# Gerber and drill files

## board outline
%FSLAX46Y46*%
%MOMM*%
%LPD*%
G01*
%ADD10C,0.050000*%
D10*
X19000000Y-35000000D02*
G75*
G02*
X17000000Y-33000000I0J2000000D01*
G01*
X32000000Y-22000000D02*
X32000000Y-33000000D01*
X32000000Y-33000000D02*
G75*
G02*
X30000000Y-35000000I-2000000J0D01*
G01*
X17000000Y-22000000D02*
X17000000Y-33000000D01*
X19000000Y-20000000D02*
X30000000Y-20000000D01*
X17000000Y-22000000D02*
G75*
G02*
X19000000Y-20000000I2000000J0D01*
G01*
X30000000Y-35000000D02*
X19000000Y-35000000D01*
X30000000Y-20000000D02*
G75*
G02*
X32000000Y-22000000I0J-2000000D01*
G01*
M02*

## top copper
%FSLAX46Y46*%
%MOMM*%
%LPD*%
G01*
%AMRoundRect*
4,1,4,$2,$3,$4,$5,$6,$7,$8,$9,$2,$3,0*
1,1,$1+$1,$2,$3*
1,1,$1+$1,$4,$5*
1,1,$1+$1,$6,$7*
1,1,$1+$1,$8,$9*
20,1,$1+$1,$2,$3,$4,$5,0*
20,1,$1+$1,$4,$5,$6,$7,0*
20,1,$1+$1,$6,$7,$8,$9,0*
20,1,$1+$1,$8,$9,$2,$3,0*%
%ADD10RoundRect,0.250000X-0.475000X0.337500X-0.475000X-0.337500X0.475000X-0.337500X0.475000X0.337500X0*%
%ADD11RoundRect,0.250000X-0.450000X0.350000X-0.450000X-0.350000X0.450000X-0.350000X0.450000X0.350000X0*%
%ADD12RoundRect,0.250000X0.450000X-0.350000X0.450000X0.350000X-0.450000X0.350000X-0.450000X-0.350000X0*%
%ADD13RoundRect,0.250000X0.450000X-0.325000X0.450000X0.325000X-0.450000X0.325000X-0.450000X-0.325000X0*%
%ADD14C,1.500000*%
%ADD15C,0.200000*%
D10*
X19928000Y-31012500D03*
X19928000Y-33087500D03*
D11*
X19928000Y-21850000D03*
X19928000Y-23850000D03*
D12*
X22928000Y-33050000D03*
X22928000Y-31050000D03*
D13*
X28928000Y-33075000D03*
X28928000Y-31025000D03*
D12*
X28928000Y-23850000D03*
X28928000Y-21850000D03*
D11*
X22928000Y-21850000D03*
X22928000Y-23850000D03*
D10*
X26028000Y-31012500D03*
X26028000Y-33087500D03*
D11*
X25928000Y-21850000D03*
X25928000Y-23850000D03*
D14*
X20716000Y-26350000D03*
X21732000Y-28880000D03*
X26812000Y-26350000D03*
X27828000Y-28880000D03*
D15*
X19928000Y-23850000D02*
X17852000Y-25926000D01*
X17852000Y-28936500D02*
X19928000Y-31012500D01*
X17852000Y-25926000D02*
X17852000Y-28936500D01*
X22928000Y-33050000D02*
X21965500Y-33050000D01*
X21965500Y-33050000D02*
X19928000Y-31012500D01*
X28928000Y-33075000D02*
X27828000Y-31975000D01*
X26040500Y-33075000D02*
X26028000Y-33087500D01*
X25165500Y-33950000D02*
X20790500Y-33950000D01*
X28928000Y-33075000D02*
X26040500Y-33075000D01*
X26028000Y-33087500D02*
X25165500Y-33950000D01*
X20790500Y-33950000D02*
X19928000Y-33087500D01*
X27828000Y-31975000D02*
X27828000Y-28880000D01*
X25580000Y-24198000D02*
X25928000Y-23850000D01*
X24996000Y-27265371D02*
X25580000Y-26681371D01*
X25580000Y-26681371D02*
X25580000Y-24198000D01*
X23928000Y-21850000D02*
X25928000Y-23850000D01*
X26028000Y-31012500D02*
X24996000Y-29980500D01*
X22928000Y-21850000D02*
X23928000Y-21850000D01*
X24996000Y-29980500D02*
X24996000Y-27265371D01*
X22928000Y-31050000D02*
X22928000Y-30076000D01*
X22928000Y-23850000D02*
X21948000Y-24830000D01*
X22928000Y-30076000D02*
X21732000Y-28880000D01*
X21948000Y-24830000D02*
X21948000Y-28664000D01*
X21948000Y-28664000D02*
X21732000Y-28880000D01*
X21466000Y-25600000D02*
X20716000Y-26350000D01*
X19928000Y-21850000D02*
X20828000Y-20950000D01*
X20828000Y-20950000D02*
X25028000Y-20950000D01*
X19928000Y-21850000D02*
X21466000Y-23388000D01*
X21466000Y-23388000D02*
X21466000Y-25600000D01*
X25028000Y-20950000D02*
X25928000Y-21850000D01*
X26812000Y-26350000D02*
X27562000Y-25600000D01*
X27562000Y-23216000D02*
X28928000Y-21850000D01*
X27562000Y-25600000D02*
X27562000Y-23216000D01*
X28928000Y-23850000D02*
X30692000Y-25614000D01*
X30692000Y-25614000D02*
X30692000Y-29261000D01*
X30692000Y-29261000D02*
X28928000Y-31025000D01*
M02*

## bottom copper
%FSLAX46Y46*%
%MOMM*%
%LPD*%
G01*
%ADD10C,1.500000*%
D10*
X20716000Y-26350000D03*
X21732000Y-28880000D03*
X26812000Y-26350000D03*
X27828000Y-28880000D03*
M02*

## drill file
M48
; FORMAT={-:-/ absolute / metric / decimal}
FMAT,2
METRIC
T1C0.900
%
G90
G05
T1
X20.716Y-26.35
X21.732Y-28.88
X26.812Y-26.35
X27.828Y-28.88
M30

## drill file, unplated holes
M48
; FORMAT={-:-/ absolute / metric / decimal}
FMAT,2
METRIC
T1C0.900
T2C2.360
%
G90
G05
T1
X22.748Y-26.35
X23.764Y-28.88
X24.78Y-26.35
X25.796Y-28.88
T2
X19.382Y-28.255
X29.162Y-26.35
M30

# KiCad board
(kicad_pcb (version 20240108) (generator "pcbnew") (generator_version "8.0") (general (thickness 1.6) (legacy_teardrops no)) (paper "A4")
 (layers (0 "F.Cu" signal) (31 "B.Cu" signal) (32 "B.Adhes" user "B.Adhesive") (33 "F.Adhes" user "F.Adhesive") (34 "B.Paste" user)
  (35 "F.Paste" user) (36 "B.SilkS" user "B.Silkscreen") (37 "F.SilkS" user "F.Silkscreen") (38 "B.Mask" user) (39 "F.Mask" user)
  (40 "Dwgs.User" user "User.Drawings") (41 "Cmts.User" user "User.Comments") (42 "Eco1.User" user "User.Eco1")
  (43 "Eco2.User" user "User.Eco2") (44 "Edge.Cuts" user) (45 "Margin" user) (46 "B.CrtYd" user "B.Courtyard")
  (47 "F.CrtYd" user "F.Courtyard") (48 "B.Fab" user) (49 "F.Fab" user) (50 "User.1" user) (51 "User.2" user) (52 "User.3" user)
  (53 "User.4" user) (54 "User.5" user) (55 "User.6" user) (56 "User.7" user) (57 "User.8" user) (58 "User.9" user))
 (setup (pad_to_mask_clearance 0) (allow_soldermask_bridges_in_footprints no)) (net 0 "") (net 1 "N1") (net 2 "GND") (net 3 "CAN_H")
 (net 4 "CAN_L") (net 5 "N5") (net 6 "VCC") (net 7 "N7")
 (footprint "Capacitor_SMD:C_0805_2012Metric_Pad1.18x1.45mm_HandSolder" (layer "F.Cu") (at 19.928 32.05 -90)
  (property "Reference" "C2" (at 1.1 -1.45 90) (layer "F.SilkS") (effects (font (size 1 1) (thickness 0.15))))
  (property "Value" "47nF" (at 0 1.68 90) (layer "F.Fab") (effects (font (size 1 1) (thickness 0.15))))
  (pad "1" smd roundrect (at -1.0375 0 270) (size 1.175 1.45) (layers "F.Cu" "F.Paste" "F.Mask") (roundrect_rratio 0.212766) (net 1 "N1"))
  (pad "2" smd roundrect (at 1.0375 0 270) (size 1.175 1.45) (layers "F.Cu" "F.Paste" "F.Mask") (roundrect_rratio 0.212766) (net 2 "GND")))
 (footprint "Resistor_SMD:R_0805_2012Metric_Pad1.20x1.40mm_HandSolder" (layer "F.Cu") (at 19.928 22.85 -90)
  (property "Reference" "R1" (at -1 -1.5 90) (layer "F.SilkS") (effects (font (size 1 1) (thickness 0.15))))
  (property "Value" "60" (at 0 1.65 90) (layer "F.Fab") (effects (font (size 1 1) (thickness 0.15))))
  (pad "1" smd roundrect (at -1 0 270) (size 1.2 1.4) (layers "F.Cu" "F.Paste" "F.Mask") (roundrect_rratio 0.208333) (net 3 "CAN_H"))
  (pad "2" smd roundrect (at 1 0 270) (size 1.2 1.4) (layers "F.Cu" "F.Paste" "F.Mask") (roundrect_rratio 0.208333) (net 1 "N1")))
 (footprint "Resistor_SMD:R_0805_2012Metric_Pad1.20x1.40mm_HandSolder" (layer "F.Cu") (at 22.928 32.05 90)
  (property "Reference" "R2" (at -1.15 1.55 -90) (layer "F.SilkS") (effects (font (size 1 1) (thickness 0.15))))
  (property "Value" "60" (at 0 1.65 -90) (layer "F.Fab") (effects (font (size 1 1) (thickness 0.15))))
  (pad "1" smd roundrect (at -1 0 90) (size 1.2 1.4) (layers "F.Cu" "F.Paste" "F.Mask") (roundrect_rratio 0.208333) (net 1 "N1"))
  (pad "2" smd roundrect (at 1 0 90) (size 1.2 1.4) (layers "F.Cu" "F.Paste" "F.Mask") (roundrect_rratio 0.208333) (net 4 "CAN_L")))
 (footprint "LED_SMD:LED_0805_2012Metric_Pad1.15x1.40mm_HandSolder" (layer "F.Cu") (at 28.928 32.05 90)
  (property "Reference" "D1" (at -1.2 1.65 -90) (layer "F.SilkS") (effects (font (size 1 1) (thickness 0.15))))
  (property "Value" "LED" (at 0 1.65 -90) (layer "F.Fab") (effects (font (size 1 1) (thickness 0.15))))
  (pad "1" smd roundrect (at -1.025 0 90) (size 1.15 1.4) (layers "F.Cu" "F.Paste" "F.Mask") (roundrect_rratio 0.217391) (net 2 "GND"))
  (pad "2" smd roundrect (at 1.025 0 90) (size 1.15 1.4) (layers "F.Cu" "F.Paste" "F.Mask") (roundrect_rratio 0.217391) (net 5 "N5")))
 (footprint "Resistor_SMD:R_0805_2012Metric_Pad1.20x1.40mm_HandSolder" (layer "F.Cu") (at 28.928 22.85 90)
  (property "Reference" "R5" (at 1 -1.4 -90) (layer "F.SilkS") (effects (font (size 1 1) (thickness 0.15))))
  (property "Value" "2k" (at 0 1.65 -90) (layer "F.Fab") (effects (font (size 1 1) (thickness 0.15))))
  (pad "1" smd roundrect (at -1 0 90) (size 1.2 1.4) (layers "F.Cu" "F.Paste" "F.Mask") (roundrect_rratio 0.208333) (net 5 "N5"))
  (pad "2" smd roundrect (at 1 0 90) (size 1.2 1.4) (layers "F.Cu" "F.Paste" "F.Mask") (roundrect_rratio 0.208333) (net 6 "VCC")))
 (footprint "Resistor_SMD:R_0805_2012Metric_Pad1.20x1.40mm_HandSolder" (layer "F.Cu") (at 22.928 22.85 -90)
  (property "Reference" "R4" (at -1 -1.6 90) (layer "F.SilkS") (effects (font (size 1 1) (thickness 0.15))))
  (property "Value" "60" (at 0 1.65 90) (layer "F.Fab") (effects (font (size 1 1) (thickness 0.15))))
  (pad "1" smd roundrect (at -1 0 270) (size 1.2 1.4) (layers "F.Cu" "F.Paste" "F.Mask") (roundrect_rratio 0.208333) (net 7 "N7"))
  (pad "2" smd roundrect (at 1 0 270) (size 1.2 1.4) (layers "F.Cu" "F.Paste" "F.Mask") (roundrect_rratio 0.208333) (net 4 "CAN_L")))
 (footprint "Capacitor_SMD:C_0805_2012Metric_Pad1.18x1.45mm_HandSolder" (layer "F.Cu") (at 26.028 32.05 -90)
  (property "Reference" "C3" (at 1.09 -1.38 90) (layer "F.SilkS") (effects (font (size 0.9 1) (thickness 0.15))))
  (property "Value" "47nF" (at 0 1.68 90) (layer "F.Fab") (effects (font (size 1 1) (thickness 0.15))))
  (pad "1" smd roundrect (at -1.0375 0 270) (size 1.175 1.45) (layers "F.Cu" "F.Paste" "F.Mask") (roundrect_rratio 0.212766) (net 7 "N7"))
  (pad "2" smd roundrect (at 1.0375 0 270) (size 1.175 1.45) (layers "F.Cu" "F.Paste" "F.Mask") (roundrect_rratio 0.212766) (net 2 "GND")))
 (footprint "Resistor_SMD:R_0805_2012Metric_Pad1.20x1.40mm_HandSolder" (layer "F.Cu") (at 25.928 22.85 -90)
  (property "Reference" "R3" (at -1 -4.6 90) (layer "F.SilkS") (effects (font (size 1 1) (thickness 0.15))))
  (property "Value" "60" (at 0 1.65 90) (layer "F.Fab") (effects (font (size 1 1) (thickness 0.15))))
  (pad "1" smd roundrect (at -1 0 270) (size 1.2 1.4) (layers "F.Cu" "F.Paste" "F.Mask") (roundrect_rratio 0.208333) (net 3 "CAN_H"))
  (pad "2" smd roundrect (at 1 0 270) (size 1.2 1.4) (layers "F.Cu" "F.Paste" "F.Mask") (roundrect_rratio 0.208333) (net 7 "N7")))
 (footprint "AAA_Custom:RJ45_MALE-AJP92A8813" (layer "B.Cu") (at 24.272 27.62 180)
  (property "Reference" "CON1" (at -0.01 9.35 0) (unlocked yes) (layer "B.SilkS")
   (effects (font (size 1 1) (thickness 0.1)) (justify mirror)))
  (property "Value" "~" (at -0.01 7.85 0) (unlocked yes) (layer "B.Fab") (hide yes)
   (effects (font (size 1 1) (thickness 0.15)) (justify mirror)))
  (pad "" np_thru_hole circle (at -4.89 1.27 180) (size 2.3 2.3) (drill 2.36) (layers "F&B.Cu" "*.Mask"))
  (pad "" np_thru_hole circle (at -1.524 -1.26 180) (size 0.9 0.9) (drill 0.9) (layers "F&B.Cu" "*.Mask"))
  (pad "" np_thru_hole circle (at -0.508 1.27 180) (size 0.9 0.9) (drill 0.9) (layers "F&B.Cu" "*.Mask"))
  (pad "" np_thru_hole circle (at 0.508 -1.26 180) (size 0.9 0.9) (drill 0.9) (layers "F&B.Cu" "*.Mask"))
  (pad "" np_thru_hole circle (at 1.524 1.27 180) (size 0.9 0.9) (drill 0.9) (layers "F&B.Cu" "*.Mask"))
  (pad "" np_thru_hole circle (at 4.89 -0.635 180) (size 2.3 2.3) (drill 2.36) (layers "F&B.Cu" "*.Mask"))
  (pad "1" thru_hole circle (at 3.556 1.27 180) (size 1.5 1.5) (drill 0.9) (layers "*.Cu" "*.Mask") (remove_unused_layers no)
   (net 3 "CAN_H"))
  (pad "2" thru_hole circle (at 2.54 -1.26 180) (size 1.5 1.5) (drill 0.9) (layers "*.Cu" "*.Mask") (remove_unused_layers no)
   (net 4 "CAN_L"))
  (pad "7" thru_hole circle (at -2.54 1.27 180) (size 1.5 1.5) (drill 0.9) (layers "*.Cu" "*.Mask") (remove_unused_layers no) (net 6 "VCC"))
  (pad "8" thru_hole circle (at -3.556 -1.26 180) (size 1.5 1.5) (drill 0.9) (layers "*.Cu" "*.Mask") (remove_unused_layers no)
   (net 2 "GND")))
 (gr_arc (start 19 35) (mid 17.585786 34.414214) (end 17 33) (stroke (width 0.05) (type default)) (layer "Edge.Cuts"))
 (gr_line (start 32 22) (end 32 33) (stroke (width 0.05) (type default)) (layer "Edge.Cuts"))
 (gr_arc (start 32 33) (mid 31.414214 34.414214) (end 30 35) (stroke (width 0.05) (type default)) (layer "Edge.Cuts"))
 (gr_line (start 17 22) (end 17 33) (stroke (width 0.05) (type default)) (layer "Edge.Cuts"))
 (gr_line (start 19 20) (end 30 20) (stroke (width 0.05) (type default)) (layer "Edge.Cuts"))
 (gr_arc (start 17 22) (mid 17.585786 20.585786) (end 19 20) (stroke (width 0.05) (type default)) (layer "Edge.Cuts"))
 (gr_line (start 30 35) (end 19 35) (stroke (width 0.05) (type default)) (layer "Edge.Cuts"))
 (gr_arc (start 30 20) (mid 31.414214 20.585786) (end 32 22) (stroke (width 0.05) (type default)) (layer "Edge.Cuts"))
 (segment (start 19.928 23.85) (end 17.852 25.926) (width 0.2) (layer "F.Cu") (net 1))
 (segment (start 17.852 28.9365) (end 19.928 31.0125) (width 0.2) (layer "F.Cu") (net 1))
 (segment (start 17.852 25.926) (end 17.852 28.9365) (width 0.2) (layer "F.Cu") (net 1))
 (segment (start 22.928 33.05) (end 21.9655 33.05) (width 0.2) (layer "F.Cu") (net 1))
 (segment (start 21.9655 33.05) (end 19.928 31.0125) (width 0.2) (layer "F.Cu") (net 1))
 (segment (start 28.928 33.075) (end 27.828 31.975) (width 0.2) (layer "F.Cu") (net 2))
 (segment (start 26.0405 33.075) (end 26.028 33.0875) (width 0.2) (layer "F.Cu") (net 2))
 (segment (start 25.1655 33.95) (end 20.7905 33.95) (width 0.2) (layer "F.Cu") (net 2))
 (segment (start 28.928 33.075) (end 26.0405 33.075) (width 0.2) (layer "F.Cu") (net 2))
 (segment (start 26.028 33.0875) (end 25.1655 33.95) (width 0.2) (layer "F.Cu") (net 2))
 (segment (start 20.7905 33.95) (end 19.928 33.0875) (width 0.2) (layer "F.Cu") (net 2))
 (segment (start 27.828 31.975) (end 27.828 28.88) (width 0.2) (layer "F.Cu") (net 2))
 (segment (start 25.58 24.198) (end 25.928 23.85) (width 0.2) (layer "F.Cu") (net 7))
 (segment (start 24.996 27.265371) (end 25.58 26.681371) (width 0.2) (layer "F.Cu") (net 7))
 (segment (start 25.58 26.681371) (end 25.58 24.198) (width 0.2) (layer "F.Cu") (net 7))
 (segment (start 23.928 21.85) (end 25.928 23.85) (width 0.2) (layer "F.Cu") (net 7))
 (segment (start 26.028 31.0125) (end 24.996 29.9805) (width 0.2) (layer "F.Cu") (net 7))
 (segment (start 22.928 21.85) (end 23.928 21.85) (width 0.2) (layer "F.Cu") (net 7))
 (segment (start 24.996 29.9805) (end 24.996 27.265371) (width 0.2) (layer "F.Cu") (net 7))
 (segment (start 22.928 31.05) (end 22.928 30.076) (width 0.2) (layer "F.Cu") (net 4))
 (segment (start 22.928 23.85) (end 21.948 24.83) (width 0.2) (layer "F.Cu") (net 4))
 (segment (start 22.928 30.076) (end 21.732 28.88) (width 0.2) (layer "F.Cu") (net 4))
 (segment (start 21.948 24.83) (end 21.948 28.664) (width 0.2) (layer "F.Cu") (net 4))
 (segment (start 21.948 28.664) (end 21.732 28.88) (width 0.2) (layer "F.Cu") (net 4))
 (segment (start 21.466 25.6) (end 20.716 26.35) (width 0.2) (layer "F.Cu") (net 3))
 (segment (start 19.928 21.85) (end 20.828 20.95) (width 0.2) (layer "F.Cu") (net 3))
 (segment (start 20.828 20.95) (end 25.028 20.95) (width 0.2) (layer "F.Cu") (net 3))
 (segment (start 19.928 21.85) (end 21.466 23.388) (width 0.2) (layer "F.Cu") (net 3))
 (segment (start 21.466 23.388) (end 21.466 25.6) (width 0.2) (layer "F.Cu") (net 3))
 (segment (start 25.028 20.95) (end 25.928 21.85) (width 0.2) (layer "F.Cu") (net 3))
 (segment (start 26.812 26.35) (end 27.562 25.6) (width 0.2) (layer "F.Cu") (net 6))
 (segment (start 27.562 23.216) (end 28.928 21.85) (width 0.2) (layer "F.Cu") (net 6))
 (segment (start 27.562 25.6) (end 27.562 23.216) (width 0.2) (layer "F.Cu") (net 6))
 (segment (start 28.928 23.85) (end 30.692 25.614) (width 0.2) (layer "F.Cu") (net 5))
 (segment (start 30.692 25.614) (end 30.692 29.261) (width 0.2) (layer "F.Cu") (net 5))
 (segment (start 30.692 29.261) (end 28.928 31.025) (width 0.2) (layer "F.Cu") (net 5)))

